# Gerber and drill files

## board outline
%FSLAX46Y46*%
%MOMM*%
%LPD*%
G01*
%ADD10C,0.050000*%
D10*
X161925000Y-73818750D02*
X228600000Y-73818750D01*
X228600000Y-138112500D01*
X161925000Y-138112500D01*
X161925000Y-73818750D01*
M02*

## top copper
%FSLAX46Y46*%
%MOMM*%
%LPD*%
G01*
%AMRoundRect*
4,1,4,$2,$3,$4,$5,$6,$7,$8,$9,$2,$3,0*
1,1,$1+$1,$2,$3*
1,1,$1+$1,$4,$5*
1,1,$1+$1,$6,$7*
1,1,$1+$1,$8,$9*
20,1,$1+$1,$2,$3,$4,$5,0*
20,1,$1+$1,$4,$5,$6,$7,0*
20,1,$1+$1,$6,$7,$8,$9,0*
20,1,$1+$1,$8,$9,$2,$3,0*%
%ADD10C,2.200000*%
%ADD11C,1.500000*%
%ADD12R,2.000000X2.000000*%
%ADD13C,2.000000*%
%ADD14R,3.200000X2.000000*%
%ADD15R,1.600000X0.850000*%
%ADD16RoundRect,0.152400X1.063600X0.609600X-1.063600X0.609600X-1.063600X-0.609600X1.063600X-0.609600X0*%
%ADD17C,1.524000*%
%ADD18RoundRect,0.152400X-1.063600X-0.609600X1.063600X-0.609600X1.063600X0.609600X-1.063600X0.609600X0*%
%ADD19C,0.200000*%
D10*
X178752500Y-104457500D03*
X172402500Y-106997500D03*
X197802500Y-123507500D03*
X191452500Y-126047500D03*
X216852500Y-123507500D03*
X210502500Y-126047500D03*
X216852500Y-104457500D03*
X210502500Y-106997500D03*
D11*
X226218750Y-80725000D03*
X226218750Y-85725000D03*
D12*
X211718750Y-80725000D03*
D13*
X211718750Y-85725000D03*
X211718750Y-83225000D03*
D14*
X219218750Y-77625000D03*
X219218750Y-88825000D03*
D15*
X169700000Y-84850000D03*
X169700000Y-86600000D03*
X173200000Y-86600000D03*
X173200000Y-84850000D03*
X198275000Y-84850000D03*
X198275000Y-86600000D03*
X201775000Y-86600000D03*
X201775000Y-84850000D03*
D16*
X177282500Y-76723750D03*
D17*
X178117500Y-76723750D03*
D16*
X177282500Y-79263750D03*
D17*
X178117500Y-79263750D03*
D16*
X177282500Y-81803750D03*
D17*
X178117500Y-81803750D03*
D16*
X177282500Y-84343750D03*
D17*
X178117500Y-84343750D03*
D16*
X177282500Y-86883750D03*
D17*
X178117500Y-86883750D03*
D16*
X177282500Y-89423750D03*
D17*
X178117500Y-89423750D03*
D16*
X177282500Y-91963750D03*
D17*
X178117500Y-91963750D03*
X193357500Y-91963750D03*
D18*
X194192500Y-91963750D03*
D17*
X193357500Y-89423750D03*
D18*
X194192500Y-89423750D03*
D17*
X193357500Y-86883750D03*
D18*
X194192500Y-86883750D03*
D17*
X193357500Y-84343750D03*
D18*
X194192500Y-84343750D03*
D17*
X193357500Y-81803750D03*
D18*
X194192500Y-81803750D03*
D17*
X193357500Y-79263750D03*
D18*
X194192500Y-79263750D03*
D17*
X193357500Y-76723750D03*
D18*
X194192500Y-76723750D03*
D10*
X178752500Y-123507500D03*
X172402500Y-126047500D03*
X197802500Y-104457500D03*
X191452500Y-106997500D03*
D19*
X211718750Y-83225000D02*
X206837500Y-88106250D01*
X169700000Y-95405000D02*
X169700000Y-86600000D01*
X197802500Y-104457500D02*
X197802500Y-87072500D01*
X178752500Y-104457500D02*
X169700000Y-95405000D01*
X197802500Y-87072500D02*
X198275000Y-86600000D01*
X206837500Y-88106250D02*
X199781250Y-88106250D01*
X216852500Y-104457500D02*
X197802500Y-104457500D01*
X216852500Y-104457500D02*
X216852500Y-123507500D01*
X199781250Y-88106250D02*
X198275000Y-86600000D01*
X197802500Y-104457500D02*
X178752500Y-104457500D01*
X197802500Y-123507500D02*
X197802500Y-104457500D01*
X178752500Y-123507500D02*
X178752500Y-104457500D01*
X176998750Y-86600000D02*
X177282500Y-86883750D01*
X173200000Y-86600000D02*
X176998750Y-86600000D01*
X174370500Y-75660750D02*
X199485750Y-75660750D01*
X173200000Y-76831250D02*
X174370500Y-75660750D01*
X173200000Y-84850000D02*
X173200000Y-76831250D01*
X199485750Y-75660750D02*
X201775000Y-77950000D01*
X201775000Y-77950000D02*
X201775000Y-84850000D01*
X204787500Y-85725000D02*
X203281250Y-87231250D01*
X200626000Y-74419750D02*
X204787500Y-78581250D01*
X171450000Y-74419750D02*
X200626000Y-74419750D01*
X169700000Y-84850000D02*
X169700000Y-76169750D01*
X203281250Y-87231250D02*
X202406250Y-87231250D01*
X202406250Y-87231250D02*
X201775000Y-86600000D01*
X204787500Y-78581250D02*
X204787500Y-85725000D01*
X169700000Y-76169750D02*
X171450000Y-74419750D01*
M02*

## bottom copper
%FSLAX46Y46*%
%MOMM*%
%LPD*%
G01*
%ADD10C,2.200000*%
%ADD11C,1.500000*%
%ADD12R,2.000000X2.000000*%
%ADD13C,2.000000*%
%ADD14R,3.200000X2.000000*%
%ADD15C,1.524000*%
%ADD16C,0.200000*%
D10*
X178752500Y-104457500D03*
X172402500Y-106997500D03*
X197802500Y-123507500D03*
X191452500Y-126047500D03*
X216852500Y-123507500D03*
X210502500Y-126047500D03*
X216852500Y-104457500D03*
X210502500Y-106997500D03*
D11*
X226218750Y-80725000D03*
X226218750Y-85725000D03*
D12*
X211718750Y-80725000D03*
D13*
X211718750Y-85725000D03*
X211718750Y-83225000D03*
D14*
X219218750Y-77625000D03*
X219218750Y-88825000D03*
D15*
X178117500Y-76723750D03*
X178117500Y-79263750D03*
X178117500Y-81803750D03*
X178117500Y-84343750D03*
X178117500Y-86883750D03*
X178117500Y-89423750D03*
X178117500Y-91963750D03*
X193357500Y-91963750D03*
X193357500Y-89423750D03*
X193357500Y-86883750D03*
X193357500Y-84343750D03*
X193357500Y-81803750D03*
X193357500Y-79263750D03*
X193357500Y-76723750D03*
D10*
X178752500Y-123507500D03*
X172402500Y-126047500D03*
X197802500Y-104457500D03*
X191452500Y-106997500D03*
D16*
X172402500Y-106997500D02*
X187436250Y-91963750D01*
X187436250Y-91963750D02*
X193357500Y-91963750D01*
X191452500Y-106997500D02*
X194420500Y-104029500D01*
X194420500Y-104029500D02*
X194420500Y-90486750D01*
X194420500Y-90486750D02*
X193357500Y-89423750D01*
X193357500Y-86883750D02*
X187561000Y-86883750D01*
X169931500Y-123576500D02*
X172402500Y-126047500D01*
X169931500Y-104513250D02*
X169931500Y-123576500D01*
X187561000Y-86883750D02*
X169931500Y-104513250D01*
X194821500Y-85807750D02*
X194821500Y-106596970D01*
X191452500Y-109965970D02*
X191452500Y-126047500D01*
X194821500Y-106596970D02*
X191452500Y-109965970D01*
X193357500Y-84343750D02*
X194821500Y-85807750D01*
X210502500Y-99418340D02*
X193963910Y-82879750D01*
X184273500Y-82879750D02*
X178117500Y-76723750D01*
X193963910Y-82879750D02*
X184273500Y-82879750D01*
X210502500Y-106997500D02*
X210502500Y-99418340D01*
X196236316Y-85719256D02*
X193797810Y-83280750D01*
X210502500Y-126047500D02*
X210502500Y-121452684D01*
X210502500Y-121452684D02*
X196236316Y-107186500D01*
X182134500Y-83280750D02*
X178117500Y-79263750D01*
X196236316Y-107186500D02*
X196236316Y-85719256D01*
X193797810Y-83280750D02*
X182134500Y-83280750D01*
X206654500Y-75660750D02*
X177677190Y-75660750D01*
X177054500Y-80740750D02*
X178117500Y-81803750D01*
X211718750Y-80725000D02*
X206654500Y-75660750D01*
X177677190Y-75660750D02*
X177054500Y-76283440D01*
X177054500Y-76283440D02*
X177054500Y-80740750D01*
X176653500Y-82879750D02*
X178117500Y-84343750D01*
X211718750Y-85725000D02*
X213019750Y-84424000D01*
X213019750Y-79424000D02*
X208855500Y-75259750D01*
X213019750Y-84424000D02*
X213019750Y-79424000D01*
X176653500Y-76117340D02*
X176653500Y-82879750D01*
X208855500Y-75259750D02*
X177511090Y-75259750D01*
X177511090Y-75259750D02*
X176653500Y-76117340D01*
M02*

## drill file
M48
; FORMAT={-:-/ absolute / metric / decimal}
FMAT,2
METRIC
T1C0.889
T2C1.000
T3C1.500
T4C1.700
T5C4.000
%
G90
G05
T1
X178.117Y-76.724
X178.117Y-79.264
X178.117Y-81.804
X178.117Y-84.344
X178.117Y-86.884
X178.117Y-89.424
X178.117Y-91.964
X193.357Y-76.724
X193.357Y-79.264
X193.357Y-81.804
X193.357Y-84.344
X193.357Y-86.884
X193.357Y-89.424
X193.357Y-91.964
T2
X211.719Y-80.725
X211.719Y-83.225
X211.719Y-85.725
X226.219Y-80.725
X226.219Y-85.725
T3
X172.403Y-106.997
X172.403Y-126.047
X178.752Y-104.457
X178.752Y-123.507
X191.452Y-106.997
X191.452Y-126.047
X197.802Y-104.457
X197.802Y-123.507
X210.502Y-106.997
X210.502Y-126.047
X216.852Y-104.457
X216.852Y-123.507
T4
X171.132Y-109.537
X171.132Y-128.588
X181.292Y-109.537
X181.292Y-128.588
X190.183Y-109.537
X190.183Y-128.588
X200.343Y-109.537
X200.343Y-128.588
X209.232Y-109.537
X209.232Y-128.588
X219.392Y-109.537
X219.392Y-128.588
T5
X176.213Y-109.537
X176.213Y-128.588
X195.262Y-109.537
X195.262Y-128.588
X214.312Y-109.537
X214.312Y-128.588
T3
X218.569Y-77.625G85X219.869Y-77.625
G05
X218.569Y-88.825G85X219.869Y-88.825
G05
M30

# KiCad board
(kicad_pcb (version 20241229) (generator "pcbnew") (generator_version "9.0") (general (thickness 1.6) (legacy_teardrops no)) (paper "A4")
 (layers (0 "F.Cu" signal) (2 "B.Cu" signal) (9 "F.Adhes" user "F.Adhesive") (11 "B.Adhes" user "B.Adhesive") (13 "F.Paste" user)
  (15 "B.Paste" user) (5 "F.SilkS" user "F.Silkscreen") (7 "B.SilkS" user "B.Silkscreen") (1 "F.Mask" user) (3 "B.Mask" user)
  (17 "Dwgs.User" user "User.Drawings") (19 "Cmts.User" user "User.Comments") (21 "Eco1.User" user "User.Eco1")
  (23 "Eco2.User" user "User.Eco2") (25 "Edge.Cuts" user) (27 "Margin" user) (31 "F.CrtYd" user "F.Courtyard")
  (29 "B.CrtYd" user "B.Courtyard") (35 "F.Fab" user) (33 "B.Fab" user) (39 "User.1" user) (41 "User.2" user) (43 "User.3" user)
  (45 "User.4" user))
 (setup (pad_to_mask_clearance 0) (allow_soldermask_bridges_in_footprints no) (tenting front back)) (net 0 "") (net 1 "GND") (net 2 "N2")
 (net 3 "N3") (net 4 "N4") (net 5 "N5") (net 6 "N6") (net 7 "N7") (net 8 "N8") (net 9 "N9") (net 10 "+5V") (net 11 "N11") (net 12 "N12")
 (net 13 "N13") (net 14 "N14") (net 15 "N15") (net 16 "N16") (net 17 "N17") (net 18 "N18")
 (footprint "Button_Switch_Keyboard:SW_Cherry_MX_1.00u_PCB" (layer "F.Cu") (at 178.7525 104.4575)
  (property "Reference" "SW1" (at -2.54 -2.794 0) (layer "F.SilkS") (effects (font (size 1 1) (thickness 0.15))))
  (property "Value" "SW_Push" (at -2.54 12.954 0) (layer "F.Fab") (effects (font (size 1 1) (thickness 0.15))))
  (pad "" np_thru_hole circle (at -7.62 5.08) (size 1.7 1.7) (drill 1.7) (layers "*.Cu" "*.Mask"))
  (pad "" np_thru_hole circle (at -2.54 5.08) (size 4 4) (drill 4) (layers "*.Cu" "*.Mask"))
  (pad "" np_thru_hole circle (at 2.54 5.08) (size 1.7 1.7) (drill 1.7) (layers "*.Cu" "*.Mask"))
  (pad "1" thru_hole circle (at 0 0) (size 2.2 2.2) (drill 1.5) (layers "*.Cu" "*.Mask") (remove_unused_layers no) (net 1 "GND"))
  (pad "2" thru_hole circle (at -6.35 2.54) (size 2.2 2.2) (drill 1.5) (layers "*.Cu" "*.Mask") (remove_unused_layers no) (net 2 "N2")))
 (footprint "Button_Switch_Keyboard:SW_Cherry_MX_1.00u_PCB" (layer "F.Cu") (at 197.8025 123.5075)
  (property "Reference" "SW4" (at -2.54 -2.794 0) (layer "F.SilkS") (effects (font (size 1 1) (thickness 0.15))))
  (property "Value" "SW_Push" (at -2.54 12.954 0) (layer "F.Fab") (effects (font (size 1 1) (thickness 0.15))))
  (pad "" np_thru_hole circle (at -7.62 5.08) (size 1.7 1.7) (drill 1.7) (layers "*.Cu" "*.Mask"))
  (pad "" np_thru_hole circle (at -2.54 5.08) (size 4 4) (drill 4) (layers "*.Cu" "*.Mask"))
  (pad "" np_thru_hole circle (at 2.54 5.08) (size 1.7 1.7) (drill 1.7) (layers "*.Cu" "*.Mask"))
  (pad "1" thru_hole circle (at 0 0) (size 2.2 2.2) (drill 1.5) (layers "*.Cu" "*.Mask") (remove_unused_layers no) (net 1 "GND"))
  (pad "2" thru_hole circle (at -6.35 2.54) (size 2.2 2.2) (drill 1.5) (layers "*.Cu" "*.Mask") (remove_unused_layers no) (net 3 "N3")))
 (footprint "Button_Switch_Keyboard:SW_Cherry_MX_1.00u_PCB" (layer "F.Cu") (at 216.8525 123.5075)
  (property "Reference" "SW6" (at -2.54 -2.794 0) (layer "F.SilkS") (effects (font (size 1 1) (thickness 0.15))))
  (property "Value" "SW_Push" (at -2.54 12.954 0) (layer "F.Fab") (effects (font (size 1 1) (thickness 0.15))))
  (pad "" np_thru_hole circle (at -7.62 5.08) (size 1.7 1.7) (drill 1.7) (layers "*.Cu" "*.Mask"))
  (pad "" np_thru_hole circle (at -2.54 5.08) (size 4 4) (drill 4) (layers "*.Cu" "*.Mask"))
  (pad "" np_thru_hole circle (at 2.54 5.08) (size 1.7 1.7) (drill 1.7) (layers "*.Cu" "*.Mask"))
  (pad "1" thru_hole circle (at 0 0) (size 2.2 2.2) (drill 1.5) (layers "*.Cu" "*.Mask") (remove_unused_layers no) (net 1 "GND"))
  (pad "2" thru_hole circle (at -6.35 2.54) (size 2.2 2.2) (drill 1.5) (layers "*.Cu" "*.Mask") (remove_unused_layers no) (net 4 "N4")))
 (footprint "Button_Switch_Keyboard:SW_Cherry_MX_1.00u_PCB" (layer "F.Cu") (at 216.8525 104.4575)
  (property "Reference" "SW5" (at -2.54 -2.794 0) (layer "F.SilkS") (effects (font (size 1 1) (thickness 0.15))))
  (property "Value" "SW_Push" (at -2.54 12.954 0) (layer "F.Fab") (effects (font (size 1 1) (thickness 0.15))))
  (pad "" np_thru_hole circle (at -7.62 5.08) (size 1.7 1.7) (drill 1.7) (layers "*.Cu" "*.Mask"))
  (pad "" np_thru_hole circle (at -2.54 5.08) (size 4 4) (drill 4) (layers "*.Cu" "*.Mask"))
  (pad "" np_thru_hole circle (at 2.54 5.08) (size 1.7 1.7) (drill 1.7) (layers "*.Cu" "*.Mask"))
  (pad "1" thru_hole circle (at 0 0) (size 2.2 2.2) (drill 1.5) (layers "*.Cu" "*.Mask") (remove_unused_layers no) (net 1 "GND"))
  (pad "2" thru_hole circle (at -6.35 2.54) (size 2.2 2.2) (drill 1.5) (layers "*.Cu" "*.Mask") (remove_unused_layers no) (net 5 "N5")))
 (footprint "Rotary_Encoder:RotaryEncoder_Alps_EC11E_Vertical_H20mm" (layer "F.Cu") (at 211.71875 80.725)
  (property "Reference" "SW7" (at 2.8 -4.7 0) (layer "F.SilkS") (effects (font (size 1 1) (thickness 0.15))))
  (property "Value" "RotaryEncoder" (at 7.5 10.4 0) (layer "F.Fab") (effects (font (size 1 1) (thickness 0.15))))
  (pad "" thru_hole circle (at 14.5 0) (size 1.5 1.5) (drill 1) (layers "*.Cu" "*.Mask") (remove_unused_layers no))
  (pad "" thru_hole circle (at 14.5 5) (size 1.5 1.5) (drill 1) (layers "*.Cu" "*.Mask") (remove_unused_layers no))
  (pad "A" thru_hole rect (at 0 0) (size 2 2) (drill 1) (layers "*.Cu" "*.Mask") (remove_unused_layers no) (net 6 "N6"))
  (pad "B" thru_hole circle (at 0 5) (size 2 2) (drill 1) (layers "*.Cu" "*.Mask") (remove_unused_layers no) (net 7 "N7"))
  (pad "C" thru_hole circle (at 0 2.5) (size 2 2) (drill 1) (layers "*.Cu" "*.Mask") (remove_unused_layers no) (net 1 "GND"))
  (pad "MP" thru_hole rect (at 7.5 -3.1) (size 3.2 2) (drill oval 2.8 1.5) (layers "*.Cu" "*.Mask") (remove_unused_layers no))
  (pad "MP" thru_hole rect (at 7.5 8.1) (size 3.2 2) (drill oval 2.8 1.5) (layers "*.Cu" "*.Mask") (remove_unused_layers no)))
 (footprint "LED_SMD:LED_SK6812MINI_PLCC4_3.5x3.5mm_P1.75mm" (layer "F.Cu") (at 171.45 85.725)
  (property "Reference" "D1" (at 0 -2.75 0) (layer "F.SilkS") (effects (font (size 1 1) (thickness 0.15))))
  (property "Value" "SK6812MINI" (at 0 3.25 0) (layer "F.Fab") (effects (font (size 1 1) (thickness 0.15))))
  (pad "1" smd rect (at -1.75 -0.875) (size 1.6 0.85) (layers "F.Cu" "F.Mask" "F.Paste") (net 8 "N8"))
  (pad "2" smd rect (at -1.75 0.875) (size 1.6 0.85) (layers "F.Cu" "F.Mask" "F.Paste") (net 1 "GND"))
  (pad "3" smd rect (at 1.75 0.875) (size 1.6 0.85) (layers "F.Cu" "F.Mask" "F.Paste") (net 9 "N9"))
  (pad "4" smd rect (at 1.75 -0.875) (size 1.6 0.85) (layers "F.Cu" "F.Mask" "F.Paste") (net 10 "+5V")))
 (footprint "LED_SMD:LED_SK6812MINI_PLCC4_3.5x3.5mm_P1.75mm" (layer "F.Cu") (at 200.025 85.725)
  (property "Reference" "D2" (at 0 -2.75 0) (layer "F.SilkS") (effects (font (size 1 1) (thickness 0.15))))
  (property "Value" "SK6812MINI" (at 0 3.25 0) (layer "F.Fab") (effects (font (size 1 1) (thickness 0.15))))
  (pad "1" smd rect (at -1.75 -0.875) (size 1.6 0.85) (layers "F.Cu" "F.Mask" "F.Paste") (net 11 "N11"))
  (pad "2" smd rect (at -1.75 0.875) (size 1.6 0.85) (layers "F.Cu" "F.Mask" "F.Paste") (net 1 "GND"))
  (pad "3" smd rect (at 1.75 0.875) (size 1.6 0.85) (layers "F.Cu" "F.Mask" "F.Paste") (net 8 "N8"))
  (pad "4" smd rect (at 1.75 -0.875) (size 1.6 0.85) (layers "F.Cu" "F.Mask" "F.Paste") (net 10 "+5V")))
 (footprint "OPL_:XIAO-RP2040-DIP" (layer "F.Cu") (at 185.7375 84.34375)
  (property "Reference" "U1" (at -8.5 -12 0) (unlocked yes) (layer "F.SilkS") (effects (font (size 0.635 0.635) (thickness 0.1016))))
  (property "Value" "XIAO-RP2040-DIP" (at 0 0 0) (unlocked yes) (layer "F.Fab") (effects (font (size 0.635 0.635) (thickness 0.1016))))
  (pad "1" smd roundrect (at -8.455 -7.62 180) (size 2.432 1.524) (layers "F.Cu" "F.Mask") (roundrect_rratio 0.1) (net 5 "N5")
   (thermal_bridge_angle 45))
  (pad "1" thru_hole circle (at -7.62 -7.62 180) (size 1.524 1.524) (drill 0.889) (layers "*.Cu" "*.Mask") (remove_unused_layers no)
   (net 5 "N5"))
  (pad "2" smd roundrect (at -8.455 -5.08 180) (size 2.432 1.524) (layers "F.Cu" "F.Mask") (roundrect_rratio 0.1) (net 4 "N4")
   (thermal_bridge_angle 45))
  (pad "2" thru_hole circle (at -7.62 -5.08 180) (size 1.524 1.524) (drill 0.889) (layers "*.Cu" "*.Mask") (remove_unused_layers no)
   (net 4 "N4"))
  (pad "3" smd roundrect (at -8.455 -2.54 180) (size 2.432 1.524) (layers "F.Cu" "F.Mask") (roundrect_rratio 0.1) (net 6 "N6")
   (thermal_bridge_angle 45))
  (pad "3" thru_hole circle (at -7.62 -2.54 180) (size 1.524 1.524) (drill 0.889) (layers "*.Cu" "*.Mask") (remove_unused_layers no)
   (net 6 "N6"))
  (pad "4" smd roundrect (at -8.455 0 180) (size 2.432 1.524) (layers "F.Cu" "F.Mask") (roundrect_rratio 0.1) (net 7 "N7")
   (thermal_bridge_angle 45))
  (pad "4" thru_hole circle (at -7.62 0 180) (size 1.524 1.524) (drill 0.889) (layers "*.Cu" "*.Mask") (remove_unused_layers no)
   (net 7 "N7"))
  (pad "5" smd roundrect (at -8.455 2.54 180) (size 2.432 1.524) (layers "F.Cu" "F.Mask") (roundrect_rratio 0.1) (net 9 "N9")
   (thermal_bridge_angle 45))
  (pad "5" thru_hole circle (at -7.62 2.54 180) (size 1.524 1.524) (drill 0.889) (layers "*.Cu" "*.Mask") (remove_unused_layers no)
   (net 9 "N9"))
  (pad "6" smd roundrect (at -8.455 5.08 180) (size 2.432 1.524) (layers "F.Cu" "F.Mask") (roundrect_rratio 0.1) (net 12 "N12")
   (thermal_bridge_angle 45))
  (pad "6" thru_hole circle (at -7.62 5.08 180) (size 1.524 1.524) (drill 0.889) (layers "*.Cu" "*.Mask") (remove_unused_layers no)
   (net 12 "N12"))
  (pad "7" smd roundrect (at -8.455 7.62 180) (size 2.432 1.524) (layers "F.Cu" "F.Mask") (roundrect_rratio 0.1) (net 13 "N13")
   (thermal_bridge_angle 45))
  (pad "7" thru_hole circle (at -7.62 7.62 180) (size 1.524 1.524) (drill 0.889) (layers "*.Cu" "*.Mask") (remove_unused_layers no)
   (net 13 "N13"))
  (pad "8" thru_hole circle (at 7.62 7.62) (size 1.524 1.524) (drill 0.889) (layers "*.Cu" "*.Mask") (remove_unused_layers no) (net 2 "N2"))
  (pad "8" smd roundrect (at 8.455 7.62) (size 2.432 1.524) (layers "F.Cu" "F.Mask") (roundrect_rratio 0.1) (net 2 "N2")
   (thermal_bridge_angle 45))
  (pad "9" thru_hole circle (at 7.62 5.08) (size 1.524 1.524) (drill 0.889) (layers "*.Cu" "*.Mask") (remove_unused_layers no)
   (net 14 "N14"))
  (pad "9" smd roundrect (at 8.455 5.08) (size 2.432 1.524) (layers "F.Cu" "F.Mask") (roundrect_rratio 0.1) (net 14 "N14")
   (thermal_bridge_angle 45))
  (pad "10" thru_hole circle (at 7.62 2.54) (size 1.524 1.524) (drill 0.889) (layers "*.Cu" "*.Mask") (remove_unused_layers no)
   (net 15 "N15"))
  (pad "10" smd roundrect (at 8.455 2.54) (size 2.432 1.524) (layers "F.Cu" "F.Mask") (roundrect_rratio 0.1) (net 15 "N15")
   (thermal_bridge_angle 45))
  (pad "11" thru_hole circle (at 7.62 0) (size 1.524 1.524) (drill 0.889) (layers "*.Cu" "*.Mask") (remove_unused_layers no) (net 3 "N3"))
  (pad "11" smd roundrect (at 8.455 0) (size 2.432 1.524) (layers "F.Cu" "F.Mask") (roundrect_rratio 0.1) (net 3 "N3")
   (thermal_bridge_angle 45))
  (pad "12" thru_hole circle (at 7.62 -2.54) (size 1.524 1.524) (drill 0.889) (layers "*.Cu" "*.Mask") (remove_unused_layers no)
   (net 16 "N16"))
  (pad "12" smd roundrect (at 8.455 -2.54) (size 2.432 1.524) (layers "F.Cu" "F.Mask") (roundrect_rratio 0.1) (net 16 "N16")
   (thermal_bridge_angle 45))
  (pad "13" thru_hole circle (at 7.62 -5.08) (size 1.524 1.524) (drill 0.889) (layers "*.Cu" "*.Mask") (remove_unused_layers no)
   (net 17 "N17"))
  (pad "13" smd roundrect (at 8.455 -5.08) (size 2.432 1.524) (layers "F.Cu" "F.Mask") (roundrect_rratio 0.1) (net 17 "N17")
   (thermal_bridge_angle 45))
  (pad "14" thru_hole circle (at 7.62 -7.62) (size 1.524 1.524) (drill 0.889) (layers "*.Cu" "*.Mask") (remove_unused_layers no)
   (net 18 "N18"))
  (pad "14" smd roundrect (at 8.455 -7.62) (size 2.432 1.524) (layers "F.Cu" "F.Mask") (roundrect_rratio 0.1) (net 18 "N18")
   (thermal_bridge_angle 45)))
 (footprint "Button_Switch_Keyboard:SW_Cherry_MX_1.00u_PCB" (layer "F.Cu") (at 178.7525 123.5075)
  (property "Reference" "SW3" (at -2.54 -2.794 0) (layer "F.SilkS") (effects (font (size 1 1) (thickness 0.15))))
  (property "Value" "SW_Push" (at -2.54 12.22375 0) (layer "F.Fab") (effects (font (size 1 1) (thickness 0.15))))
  (pad "" np_thru_hole circle (at -7.62 5.08) (size 1.7 1.7) (drill 1.7) (layers "*.Cu" "*.Mask"))
  (pad "" np_thru_hole circle (at -2.54 5.08) (size 4 4) (drill 4) (layers "*.Cu" "*.Mask"))
  (pad "" np_thru_hole circle (at 2.54 5.08) (size 1.7 1.7) (drill 1.7) (layers "*.Cu" "*.Mask"))
  (pad "1" thru_hole circle (at 0 0) (size 2.2 2.2) (drill 1.5) (layers "*.Cu" "*.Mask") (remove_unused_layers no) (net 1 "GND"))
  (pad "2" thru_hole circle (at -6.35 2.54) (size 2.2 2.2) (drill 1.5) (layers "*.Cu" "*.Mask") (remove_unused_layers no) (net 15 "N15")))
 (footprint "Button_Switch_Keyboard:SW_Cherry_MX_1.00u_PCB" (layer "F.Cu") (at 197.8025 104.4575)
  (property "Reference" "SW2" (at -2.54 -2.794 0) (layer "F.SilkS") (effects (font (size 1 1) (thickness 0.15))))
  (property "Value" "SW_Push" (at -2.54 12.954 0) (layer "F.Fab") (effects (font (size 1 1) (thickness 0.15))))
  (pad "" np_thru_hole circle (at -7.62 5.08) (size 1.7 1.7) (drill 1.7) (layers "*.Cu" "*.Mask"))
  (pad "" np_thru_hole circle (at -2.54 5.08) (size 4 4) (drill 4) (layers "*.Cu" "*.Mask"))
  (pad "" np_thru_hole circle (at 2.54 5.08) (size 1.7 1.7) (drill 1.7) (layers "*.Cu" "*.Mask"))
  (pad "1" thru_hole circle (at 0 0) (size 2.2 2.2) (drill 1.5) (layers "*.Cu" "*.Mask") (remove_unused_layers no) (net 1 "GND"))
  (pad "2" thru_hole circle (at -6.35 2.54) (size 2.2 2.2) (drill 1.5) (layers "*.Cu" "*.Mask") (remove_unused_layers no) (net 14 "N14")))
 (gr_rect (start 161.925 73.81875) (end 228.6 138.1125) (stroke (width 0.05) (type default)) (fill no) (layer "Edge.Cuts"))
 (segment (start 211.71875 83.225) (end 206.8375 88.10625) (width 0.2) (layer "F.Cu") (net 1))
 (segment (start 169.7 95.405) (end 169.7 86.6) (width 0.2) (layer "F.Cu") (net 1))
 (segment (start 197.8025 104.4575) (end 197.8025 87.0725) (width 0.2) (layer "F.Cu") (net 1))
 (segment (start 178.7525 104.4575) (end 169.7 95.405) (width 0.2) (layer "F.Cu") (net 1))
 (segment (start 197.8025 87.0725) (end 198.275 86.6) (width 0.2) (layer "F.Cu") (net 1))
 (segment (start 206.8375 88.10625) (end 199.78125 88.10625) (width 0.2) (layer "F.Cu") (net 1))
 (segment (start 216.8525 104.4575) (end 197.8025 104.4575) (width 0.2) (layer "F.Cu") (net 1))
 (segment (start 216.8525 104.4575) (end 216.8525 123.5075) (width 0.2) (layer "F.Cu") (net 1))
 (segment (start 199.78125 88.10625) (end 198.275 86.6) (width 0.2) (layer "F.Cu") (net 1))
 (segment (start 197.8025 104.4575) (end 178.7525 104.4575) (width 0.2) (layer "F.Cu") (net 1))
 (segment (start 197.8025 123.5075) (end 197.8025 104.4575) (width 0.2) (layer "F.Cu") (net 1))
 (segment (start 178.7525 123.5075) (end 178.7525 104.4575) (width 0.2) (layer "F.Cu") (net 1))
 (segment (start 176.99875 86.6) (end 177.2825 86.88375) (width 0.2) (layer "F.Cu") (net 9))
 (segment (start 173.2 86.6) (end 176.99875 86.6) (width 0.2) (layer "F.Cu") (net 9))
 (segment (start 174.3705 75.66075) (end 199.48575 75.66075) (width 0.2) (layer "F.Cu") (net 10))
 (segment (start 173.2 76.83125) (end 174.3705 75.66075) (width 0.2) (layer "F.Cu") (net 10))
 (segment (start 173.2 84.85) (end 173.2 76.83125) (width 0.2) (layer "F.Cu") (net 10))
 (segment (start 199.48575 75.66075) (end 201.775 77.95) (width 0.2) (layer "F.Cu") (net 10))
 (segment (start 201.775 77.95) (end 201.775 84.85) (width 0.2) (layer "F.Cu") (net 10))
 (segment (start 204.7875 85.725) (end 203.28125 87.23125) (width 0.2) (layer "F.Cu") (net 8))
 (segment (start 200.626 74.41975) (end 204.7875 78.58125) (width 0.2) (layer "F.Cu") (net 8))
 (segment (start 171.45 74.41975) (end 200.626 74.41975) (width 0.2) (layer "F.Cu") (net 8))
 (segment (start 169.7 84.85) (end 169.7 76.16975) (width 0.2) (layer "F.Cu") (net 8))
 (segment (start 203.28125 87.23125) (end 202.40625 87.23125) (width 0.2) (layer "F.Cu") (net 8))
 (segment (start 202.40625 87.23125) (end 201.775 86.6) (width 0.2) (layer "F.Cu") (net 8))
 (segment (start 204.7875 78.58125) (end 204.7875 85.725) (width 0.2) (layer "F.Cu") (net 8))
 (segment (start 169.7 76.16975) (end 171.45 74.41975) (width 0.2) (layer "F.Cu") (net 8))
 (segment (start 172.4025 106.9975) (end 187.43625 91.96375) (width 0.2) (layer "B.Cu") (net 2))
 (segment (start 187.43625 91.96375) (end 193.3575 91.96375) (width 0.2) (layer "B.Cu") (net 2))
 (segment (start 191.4525 106.9975) (end 194.4205 104.0295) (width 0.2) (layer "B.Cu") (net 14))
 (segment (start 194.4205 104.0295) (end 194.4205 90.48675) (width 0.2) (layer "B.Cu") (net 14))
 (segment (start 194.4205 90.48675) (end 193.3575 89.42375) (width 0.2) (layer "B.Cu") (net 14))
 (segment (start 193.3575 86.88375) (end 187.561 86.88375) (width 0.2) (layer "B.Cu") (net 15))
 (segment (start 169.9315 123.5765) (end 172.4025 126.0475) (width 0.2) (layer "B.Cu") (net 15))
 (segment (start 169.9315 104.51325) (end 169.9315 123.5765) (width 0.2) (layer "B.Cu") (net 15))
 (segment (start 187.561 86.88375) (end 169.9315 104.51325) (width 0.2) (layer "B.Cu") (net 15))
 (segment (start 194.8215 85.80775) (end 194.8215 106.59697) (width 0.2) (layer "B.Cu") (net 3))
 (segment (start 191.4525 109.96597) (end 191.4525 126.0475) (width 0.2) (layer "B.Cu") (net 3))
 (segment (start 194.8215 106.59697) (end 191.4525 109.96597) (width 0.2) (layer "B.Cu") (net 3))
 (segment (start 193.3575 84.34375) (end 194.8215 85.80775) (width 0.2) (layer "B.Cu") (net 3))
 (segment (start 210.5025 99.41834) (end 193.96391 82.87975) (width 0.2) (layer "B.Cu") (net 5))
 (segment (start 184.2735 82.87975) (end 178.1175 76.72375) (width 0.2) (layer "B.Cu") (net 5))
 (segment (start 193.96391 82.87975) (end 184.2735 82.87975) (width 0.2) (layer "B.Cu") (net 5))
 (segment (start 210.5025 106.9975) (end 210.5025 99.41834) (width 0.2) (layer "B.Cu") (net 5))
 (segment (start 196.236316 85.719256) (end 193.79781 83.28075) (width 0.2) (layer "B.Cu") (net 4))
 (segment (start 210.5025 126.0475) (end 210.5025 121.452684) (width 0.2) (layer "B.Cu") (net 4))
 (segment (start 210.5025 121.452684) (end 196.236316 107.1865) (width 0.2) (layer "B.Cu") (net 4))
 (segment (start 182.1345 83.28075) (end 178.1175 79.26375) (width 0.2) (layer "B.Cu") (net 4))
 (segment (start 196.236316 107.1865) (end 196.236316 85.719256) (width 0.2) (layer "B.Cu") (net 4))
 (segment (start 193.79781 83.28075) (end 182.1345 83.28075) (width 0.2) (layer "B.Cu") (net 4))
 (segment (start 206.6545 75.66075) (end 177.67719 75.66075) (width 0.2) (layer "B.Cu") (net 6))
 (segment (start 177.0545 80.74075) (end 178.1175 81.80375) (width 0.2) (layer "B.Cu") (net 6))
 (segment (start 211.71875 80.725) (end 206.6545 75.66075) (width 0.2) (layer "B.Cu") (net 6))
 (segment (start 177.67719 75.66075) (end 177.0545 76.28344) (width 0.2) (layer "B.Cu") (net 6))
 (segment (start 177.0545 76.28344) (end 177.0545 80.74075) (width 0.2) (layer "B.Cu") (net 6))
 (segment (start 176.6535 82.87975) (end 178.1175 84.34375) (width 0.2) (layer "B.Cu") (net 7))
 (segment (start 211.71875 85.725) (end 213.01975 84.424) (width 0.2) (layer "B.Cu") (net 7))
 (segment (start 213.01975 79.424) (end 208.8555 75.25975) (width 0.2) (layer "B.Cu") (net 7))
 (segment (start 213.01975 84.424) (end 213.01975 79.424) (width 0.2) (layer "B.Cu") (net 7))
 (segment (start 176.6535 76.11734) (end 176.6535 82.87975) (width 0.2) (layer "B.Cu") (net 7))
 (segment (start 208.8555 75.25975) (end 177.51109 75.25975) (width 0.2) (layer "B.Cu") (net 7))
 (segment (start 177.51109 75.25975) (end 176.6535 76.11734) (width 0.2) (layer "B.Cu") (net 7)))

